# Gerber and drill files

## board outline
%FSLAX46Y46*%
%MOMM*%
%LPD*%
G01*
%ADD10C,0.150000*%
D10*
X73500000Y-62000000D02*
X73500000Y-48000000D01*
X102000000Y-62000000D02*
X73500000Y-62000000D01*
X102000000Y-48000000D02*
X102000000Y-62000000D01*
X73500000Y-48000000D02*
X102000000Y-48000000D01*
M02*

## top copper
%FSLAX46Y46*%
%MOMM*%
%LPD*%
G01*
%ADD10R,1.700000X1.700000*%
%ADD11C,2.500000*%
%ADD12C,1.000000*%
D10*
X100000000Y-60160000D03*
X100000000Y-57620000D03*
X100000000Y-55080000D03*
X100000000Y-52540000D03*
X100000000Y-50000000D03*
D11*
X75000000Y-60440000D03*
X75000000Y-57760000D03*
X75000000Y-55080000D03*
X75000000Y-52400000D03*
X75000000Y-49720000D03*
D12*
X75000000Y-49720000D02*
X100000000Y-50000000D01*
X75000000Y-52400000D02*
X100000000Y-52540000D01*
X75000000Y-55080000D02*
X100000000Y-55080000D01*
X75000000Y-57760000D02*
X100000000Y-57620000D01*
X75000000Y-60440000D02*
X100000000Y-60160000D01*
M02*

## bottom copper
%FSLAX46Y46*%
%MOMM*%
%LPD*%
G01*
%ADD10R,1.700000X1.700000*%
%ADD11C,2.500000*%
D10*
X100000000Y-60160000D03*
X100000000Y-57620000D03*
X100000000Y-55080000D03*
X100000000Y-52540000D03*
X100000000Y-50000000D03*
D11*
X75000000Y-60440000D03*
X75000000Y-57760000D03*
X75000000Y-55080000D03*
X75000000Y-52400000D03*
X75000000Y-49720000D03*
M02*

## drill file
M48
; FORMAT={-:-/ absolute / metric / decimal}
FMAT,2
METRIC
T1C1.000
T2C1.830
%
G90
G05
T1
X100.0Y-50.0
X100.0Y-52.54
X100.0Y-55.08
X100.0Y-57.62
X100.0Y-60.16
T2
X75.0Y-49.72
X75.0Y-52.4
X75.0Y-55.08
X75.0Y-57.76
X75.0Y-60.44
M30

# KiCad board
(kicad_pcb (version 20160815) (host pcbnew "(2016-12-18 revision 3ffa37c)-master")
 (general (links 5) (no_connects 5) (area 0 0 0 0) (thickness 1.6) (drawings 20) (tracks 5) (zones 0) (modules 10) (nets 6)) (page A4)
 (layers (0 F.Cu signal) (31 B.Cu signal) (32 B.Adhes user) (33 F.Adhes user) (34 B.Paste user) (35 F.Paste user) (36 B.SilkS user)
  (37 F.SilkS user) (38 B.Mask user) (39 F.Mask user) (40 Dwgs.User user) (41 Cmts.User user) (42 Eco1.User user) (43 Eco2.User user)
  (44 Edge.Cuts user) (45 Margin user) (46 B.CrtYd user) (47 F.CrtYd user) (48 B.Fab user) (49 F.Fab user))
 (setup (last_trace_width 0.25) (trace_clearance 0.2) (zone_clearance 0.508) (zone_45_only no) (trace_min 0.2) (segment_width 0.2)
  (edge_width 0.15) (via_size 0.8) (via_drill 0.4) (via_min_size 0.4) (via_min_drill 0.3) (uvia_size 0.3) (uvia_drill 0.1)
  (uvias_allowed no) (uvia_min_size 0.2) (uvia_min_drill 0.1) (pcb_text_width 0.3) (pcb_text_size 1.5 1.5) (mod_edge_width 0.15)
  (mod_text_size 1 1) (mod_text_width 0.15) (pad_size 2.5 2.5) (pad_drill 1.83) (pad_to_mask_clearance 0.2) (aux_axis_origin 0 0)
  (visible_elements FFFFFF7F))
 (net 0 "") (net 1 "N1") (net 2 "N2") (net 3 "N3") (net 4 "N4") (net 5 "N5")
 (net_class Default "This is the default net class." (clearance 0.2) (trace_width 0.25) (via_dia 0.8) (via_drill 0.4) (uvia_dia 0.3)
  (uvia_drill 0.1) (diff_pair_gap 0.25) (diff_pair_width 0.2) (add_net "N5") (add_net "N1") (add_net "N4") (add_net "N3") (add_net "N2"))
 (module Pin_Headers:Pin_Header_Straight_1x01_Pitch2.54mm (layer F.Cu) (at 100 60.16)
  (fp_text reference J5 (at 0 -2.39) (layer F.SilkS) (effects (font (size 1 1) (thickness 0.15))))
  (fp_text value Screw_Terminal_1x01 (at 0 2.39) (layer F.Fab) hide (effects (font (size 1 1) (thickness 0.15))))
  (pad 1 thru_hole rect (at 0 0) (size 1.7 1.7) (drill 1) (layers *.Cu *.Mask) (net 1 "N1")))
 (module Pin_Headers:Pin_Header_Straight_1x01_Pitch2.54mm (layer F.Cu) (at 100 57.62)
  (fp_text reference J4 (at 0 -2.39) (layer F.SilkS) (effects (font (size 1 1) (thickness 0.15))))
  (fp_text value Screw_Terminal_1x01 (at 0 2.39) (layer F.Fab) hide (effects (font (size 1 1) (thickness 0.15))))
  (pad 1 thru_hole rect (at 0 0) (size 1.7 1.7) (drill 1) (layers *.Cu *.Mask) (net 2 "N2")))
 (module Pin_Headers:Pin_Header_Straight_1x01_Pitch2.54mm (layer F.Cu) (at 100 55.08)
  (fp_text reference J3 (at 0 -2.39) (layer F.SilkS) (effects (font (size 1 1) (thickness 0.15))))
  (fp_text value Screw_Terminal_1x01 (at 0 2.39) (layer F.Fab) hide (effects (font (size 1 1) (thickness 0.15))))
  (pad 1 thru_hole rect (at 0 0) (size 1.7 1.7) (drill 1) (layers *.Cu *.Mask) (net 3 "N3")))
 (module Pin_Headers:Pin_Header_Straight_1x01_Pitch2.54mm (layer F.Cu) (at 100 52.54)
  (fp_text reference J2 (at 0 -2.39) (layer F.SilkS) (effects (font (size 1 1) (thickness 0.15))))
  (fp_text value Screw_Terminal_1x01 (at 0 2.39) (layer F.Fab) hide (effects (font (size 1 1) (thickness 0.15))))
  (pad 1 thru_hole rect (at 0 0) (size 1.7 1.7) (drill 1) (layers *.Cu *.Mask) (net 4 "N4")))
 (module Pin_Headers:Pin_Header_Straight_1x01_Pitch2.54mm (layer F.Cu) (at 100 50)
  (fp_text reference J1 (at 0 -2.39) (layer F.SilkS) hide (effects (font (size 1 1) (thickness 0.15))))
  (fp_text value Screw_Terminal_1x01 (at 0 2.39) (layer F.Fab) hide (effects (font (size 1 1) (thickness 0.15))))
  (pad 1 thru_hole rect (at 0 0) (size 1.7 1.7) (drill 1) (layers *.Cu *.Mask) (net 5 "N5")))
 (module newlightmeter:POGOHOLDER (layer F.Cu) (at 91.98 66.07)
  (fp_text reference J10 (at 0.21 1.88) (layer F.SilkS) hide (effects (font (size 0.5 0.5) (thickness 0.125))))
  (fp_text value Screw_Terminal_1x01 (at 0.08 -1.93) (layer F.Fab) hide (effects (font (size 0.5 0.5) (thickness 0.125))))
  (pad 1 thru_hole circle (at -16.98 -5.63) (size 2.5 2.5) (drill 1.83) (layers *.Cu *.Mask) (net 1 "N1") (solder_mask_margin 0.05)))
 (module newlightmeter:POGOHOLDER (layer F.Cu) (at 91.56 61.63)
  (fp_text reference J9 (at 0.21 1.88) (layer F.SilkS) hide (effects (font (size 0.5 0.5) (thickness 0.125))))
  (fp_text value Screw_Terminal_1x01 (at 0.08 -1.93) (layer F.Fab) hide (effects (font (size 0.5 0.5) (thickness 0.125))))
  (pad 1 thru_hole circle (at -16.56 -3.87) (size 2.5 2.5) (drill 1.83) (layers *.Cu *.Mask) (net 2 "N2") (solder_mask_margin 0.05)))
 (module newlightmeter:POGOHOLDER (layer F.Cu) (at 91.63 57.82)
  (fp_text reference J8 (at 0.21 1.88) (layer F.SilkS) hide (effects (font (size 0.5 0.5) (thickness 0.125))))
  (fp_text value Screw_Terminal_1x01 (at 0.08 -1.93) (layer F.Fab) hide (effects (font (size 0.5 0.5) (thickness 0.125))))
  (pad 1 thru_hole circle (at -16.63 -2.74) (size 2.5 2.5) (drill 1.83) (layers *.Cu *.Mask) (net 3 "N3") (solder_mask_margin 0.05)))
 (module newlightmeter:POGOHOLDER (layer F.Cu) (at 91.65 52.4)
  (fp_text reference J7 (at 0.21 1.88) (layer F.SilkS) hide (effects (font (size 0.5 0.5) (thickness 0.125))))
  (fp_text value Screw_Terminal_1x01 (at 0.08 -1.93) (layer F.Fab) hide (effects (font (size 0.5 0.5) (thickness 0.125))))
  (pad 1 thru_hole circle (at -16.65 0) (size 2.5 2.5) (drill 1.83) (layers *.Cu *.Mask) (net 4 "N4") (solder_mask_margin 0.05)))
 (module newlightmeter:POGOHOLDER (layer F.Cu) (at 91.89 47.64)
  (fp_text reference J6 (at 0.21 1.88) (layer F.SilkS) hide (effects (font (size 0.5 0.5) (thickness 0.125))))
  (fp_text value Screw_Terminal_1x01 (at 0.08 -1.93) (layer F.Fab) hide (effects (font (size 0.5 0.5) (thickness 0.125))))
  (pad 1 thru_hole circle (at -16.89 2.08) (size 2.5 2.5) (drill 1.83) (layers *.Cu *.Mask) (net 5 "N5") (solder_mask_margin 0.05)))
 (gr_line (start 73.5 62) (end 73.5 48) (layer Edge.Cuts) (width 0.15))
 (gr_line (start 102 62) (end 73.5 62) (layer Edge.Cuts) (width 0.15))
 (gr_line (start 102 48) (end 102 62) (layer Edge.Cuts) (width 0.15))
 (gr_line (start 73.5 48) (end 102 48) (layer Edge.Cuts) (width 0.15))
 (segment (start 75 49.72) (end 100 50) (width 1) (layer F.Cu) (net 5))
 (segment (start 75 52.4) (end 100 52.54) (width 1) (layer F.Cu) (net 4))
 (segment (start 75 55.08) (end 100 55.08) (width 1) (layer F.Cu) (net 3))
 (segment (start 75 57.76) (end 100 57.62) (width 1) (layer F.Cu) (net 2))
 (segment (start 75 60.44) (end 100 60.16) (width 1) (layer F.Cu) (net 1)))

